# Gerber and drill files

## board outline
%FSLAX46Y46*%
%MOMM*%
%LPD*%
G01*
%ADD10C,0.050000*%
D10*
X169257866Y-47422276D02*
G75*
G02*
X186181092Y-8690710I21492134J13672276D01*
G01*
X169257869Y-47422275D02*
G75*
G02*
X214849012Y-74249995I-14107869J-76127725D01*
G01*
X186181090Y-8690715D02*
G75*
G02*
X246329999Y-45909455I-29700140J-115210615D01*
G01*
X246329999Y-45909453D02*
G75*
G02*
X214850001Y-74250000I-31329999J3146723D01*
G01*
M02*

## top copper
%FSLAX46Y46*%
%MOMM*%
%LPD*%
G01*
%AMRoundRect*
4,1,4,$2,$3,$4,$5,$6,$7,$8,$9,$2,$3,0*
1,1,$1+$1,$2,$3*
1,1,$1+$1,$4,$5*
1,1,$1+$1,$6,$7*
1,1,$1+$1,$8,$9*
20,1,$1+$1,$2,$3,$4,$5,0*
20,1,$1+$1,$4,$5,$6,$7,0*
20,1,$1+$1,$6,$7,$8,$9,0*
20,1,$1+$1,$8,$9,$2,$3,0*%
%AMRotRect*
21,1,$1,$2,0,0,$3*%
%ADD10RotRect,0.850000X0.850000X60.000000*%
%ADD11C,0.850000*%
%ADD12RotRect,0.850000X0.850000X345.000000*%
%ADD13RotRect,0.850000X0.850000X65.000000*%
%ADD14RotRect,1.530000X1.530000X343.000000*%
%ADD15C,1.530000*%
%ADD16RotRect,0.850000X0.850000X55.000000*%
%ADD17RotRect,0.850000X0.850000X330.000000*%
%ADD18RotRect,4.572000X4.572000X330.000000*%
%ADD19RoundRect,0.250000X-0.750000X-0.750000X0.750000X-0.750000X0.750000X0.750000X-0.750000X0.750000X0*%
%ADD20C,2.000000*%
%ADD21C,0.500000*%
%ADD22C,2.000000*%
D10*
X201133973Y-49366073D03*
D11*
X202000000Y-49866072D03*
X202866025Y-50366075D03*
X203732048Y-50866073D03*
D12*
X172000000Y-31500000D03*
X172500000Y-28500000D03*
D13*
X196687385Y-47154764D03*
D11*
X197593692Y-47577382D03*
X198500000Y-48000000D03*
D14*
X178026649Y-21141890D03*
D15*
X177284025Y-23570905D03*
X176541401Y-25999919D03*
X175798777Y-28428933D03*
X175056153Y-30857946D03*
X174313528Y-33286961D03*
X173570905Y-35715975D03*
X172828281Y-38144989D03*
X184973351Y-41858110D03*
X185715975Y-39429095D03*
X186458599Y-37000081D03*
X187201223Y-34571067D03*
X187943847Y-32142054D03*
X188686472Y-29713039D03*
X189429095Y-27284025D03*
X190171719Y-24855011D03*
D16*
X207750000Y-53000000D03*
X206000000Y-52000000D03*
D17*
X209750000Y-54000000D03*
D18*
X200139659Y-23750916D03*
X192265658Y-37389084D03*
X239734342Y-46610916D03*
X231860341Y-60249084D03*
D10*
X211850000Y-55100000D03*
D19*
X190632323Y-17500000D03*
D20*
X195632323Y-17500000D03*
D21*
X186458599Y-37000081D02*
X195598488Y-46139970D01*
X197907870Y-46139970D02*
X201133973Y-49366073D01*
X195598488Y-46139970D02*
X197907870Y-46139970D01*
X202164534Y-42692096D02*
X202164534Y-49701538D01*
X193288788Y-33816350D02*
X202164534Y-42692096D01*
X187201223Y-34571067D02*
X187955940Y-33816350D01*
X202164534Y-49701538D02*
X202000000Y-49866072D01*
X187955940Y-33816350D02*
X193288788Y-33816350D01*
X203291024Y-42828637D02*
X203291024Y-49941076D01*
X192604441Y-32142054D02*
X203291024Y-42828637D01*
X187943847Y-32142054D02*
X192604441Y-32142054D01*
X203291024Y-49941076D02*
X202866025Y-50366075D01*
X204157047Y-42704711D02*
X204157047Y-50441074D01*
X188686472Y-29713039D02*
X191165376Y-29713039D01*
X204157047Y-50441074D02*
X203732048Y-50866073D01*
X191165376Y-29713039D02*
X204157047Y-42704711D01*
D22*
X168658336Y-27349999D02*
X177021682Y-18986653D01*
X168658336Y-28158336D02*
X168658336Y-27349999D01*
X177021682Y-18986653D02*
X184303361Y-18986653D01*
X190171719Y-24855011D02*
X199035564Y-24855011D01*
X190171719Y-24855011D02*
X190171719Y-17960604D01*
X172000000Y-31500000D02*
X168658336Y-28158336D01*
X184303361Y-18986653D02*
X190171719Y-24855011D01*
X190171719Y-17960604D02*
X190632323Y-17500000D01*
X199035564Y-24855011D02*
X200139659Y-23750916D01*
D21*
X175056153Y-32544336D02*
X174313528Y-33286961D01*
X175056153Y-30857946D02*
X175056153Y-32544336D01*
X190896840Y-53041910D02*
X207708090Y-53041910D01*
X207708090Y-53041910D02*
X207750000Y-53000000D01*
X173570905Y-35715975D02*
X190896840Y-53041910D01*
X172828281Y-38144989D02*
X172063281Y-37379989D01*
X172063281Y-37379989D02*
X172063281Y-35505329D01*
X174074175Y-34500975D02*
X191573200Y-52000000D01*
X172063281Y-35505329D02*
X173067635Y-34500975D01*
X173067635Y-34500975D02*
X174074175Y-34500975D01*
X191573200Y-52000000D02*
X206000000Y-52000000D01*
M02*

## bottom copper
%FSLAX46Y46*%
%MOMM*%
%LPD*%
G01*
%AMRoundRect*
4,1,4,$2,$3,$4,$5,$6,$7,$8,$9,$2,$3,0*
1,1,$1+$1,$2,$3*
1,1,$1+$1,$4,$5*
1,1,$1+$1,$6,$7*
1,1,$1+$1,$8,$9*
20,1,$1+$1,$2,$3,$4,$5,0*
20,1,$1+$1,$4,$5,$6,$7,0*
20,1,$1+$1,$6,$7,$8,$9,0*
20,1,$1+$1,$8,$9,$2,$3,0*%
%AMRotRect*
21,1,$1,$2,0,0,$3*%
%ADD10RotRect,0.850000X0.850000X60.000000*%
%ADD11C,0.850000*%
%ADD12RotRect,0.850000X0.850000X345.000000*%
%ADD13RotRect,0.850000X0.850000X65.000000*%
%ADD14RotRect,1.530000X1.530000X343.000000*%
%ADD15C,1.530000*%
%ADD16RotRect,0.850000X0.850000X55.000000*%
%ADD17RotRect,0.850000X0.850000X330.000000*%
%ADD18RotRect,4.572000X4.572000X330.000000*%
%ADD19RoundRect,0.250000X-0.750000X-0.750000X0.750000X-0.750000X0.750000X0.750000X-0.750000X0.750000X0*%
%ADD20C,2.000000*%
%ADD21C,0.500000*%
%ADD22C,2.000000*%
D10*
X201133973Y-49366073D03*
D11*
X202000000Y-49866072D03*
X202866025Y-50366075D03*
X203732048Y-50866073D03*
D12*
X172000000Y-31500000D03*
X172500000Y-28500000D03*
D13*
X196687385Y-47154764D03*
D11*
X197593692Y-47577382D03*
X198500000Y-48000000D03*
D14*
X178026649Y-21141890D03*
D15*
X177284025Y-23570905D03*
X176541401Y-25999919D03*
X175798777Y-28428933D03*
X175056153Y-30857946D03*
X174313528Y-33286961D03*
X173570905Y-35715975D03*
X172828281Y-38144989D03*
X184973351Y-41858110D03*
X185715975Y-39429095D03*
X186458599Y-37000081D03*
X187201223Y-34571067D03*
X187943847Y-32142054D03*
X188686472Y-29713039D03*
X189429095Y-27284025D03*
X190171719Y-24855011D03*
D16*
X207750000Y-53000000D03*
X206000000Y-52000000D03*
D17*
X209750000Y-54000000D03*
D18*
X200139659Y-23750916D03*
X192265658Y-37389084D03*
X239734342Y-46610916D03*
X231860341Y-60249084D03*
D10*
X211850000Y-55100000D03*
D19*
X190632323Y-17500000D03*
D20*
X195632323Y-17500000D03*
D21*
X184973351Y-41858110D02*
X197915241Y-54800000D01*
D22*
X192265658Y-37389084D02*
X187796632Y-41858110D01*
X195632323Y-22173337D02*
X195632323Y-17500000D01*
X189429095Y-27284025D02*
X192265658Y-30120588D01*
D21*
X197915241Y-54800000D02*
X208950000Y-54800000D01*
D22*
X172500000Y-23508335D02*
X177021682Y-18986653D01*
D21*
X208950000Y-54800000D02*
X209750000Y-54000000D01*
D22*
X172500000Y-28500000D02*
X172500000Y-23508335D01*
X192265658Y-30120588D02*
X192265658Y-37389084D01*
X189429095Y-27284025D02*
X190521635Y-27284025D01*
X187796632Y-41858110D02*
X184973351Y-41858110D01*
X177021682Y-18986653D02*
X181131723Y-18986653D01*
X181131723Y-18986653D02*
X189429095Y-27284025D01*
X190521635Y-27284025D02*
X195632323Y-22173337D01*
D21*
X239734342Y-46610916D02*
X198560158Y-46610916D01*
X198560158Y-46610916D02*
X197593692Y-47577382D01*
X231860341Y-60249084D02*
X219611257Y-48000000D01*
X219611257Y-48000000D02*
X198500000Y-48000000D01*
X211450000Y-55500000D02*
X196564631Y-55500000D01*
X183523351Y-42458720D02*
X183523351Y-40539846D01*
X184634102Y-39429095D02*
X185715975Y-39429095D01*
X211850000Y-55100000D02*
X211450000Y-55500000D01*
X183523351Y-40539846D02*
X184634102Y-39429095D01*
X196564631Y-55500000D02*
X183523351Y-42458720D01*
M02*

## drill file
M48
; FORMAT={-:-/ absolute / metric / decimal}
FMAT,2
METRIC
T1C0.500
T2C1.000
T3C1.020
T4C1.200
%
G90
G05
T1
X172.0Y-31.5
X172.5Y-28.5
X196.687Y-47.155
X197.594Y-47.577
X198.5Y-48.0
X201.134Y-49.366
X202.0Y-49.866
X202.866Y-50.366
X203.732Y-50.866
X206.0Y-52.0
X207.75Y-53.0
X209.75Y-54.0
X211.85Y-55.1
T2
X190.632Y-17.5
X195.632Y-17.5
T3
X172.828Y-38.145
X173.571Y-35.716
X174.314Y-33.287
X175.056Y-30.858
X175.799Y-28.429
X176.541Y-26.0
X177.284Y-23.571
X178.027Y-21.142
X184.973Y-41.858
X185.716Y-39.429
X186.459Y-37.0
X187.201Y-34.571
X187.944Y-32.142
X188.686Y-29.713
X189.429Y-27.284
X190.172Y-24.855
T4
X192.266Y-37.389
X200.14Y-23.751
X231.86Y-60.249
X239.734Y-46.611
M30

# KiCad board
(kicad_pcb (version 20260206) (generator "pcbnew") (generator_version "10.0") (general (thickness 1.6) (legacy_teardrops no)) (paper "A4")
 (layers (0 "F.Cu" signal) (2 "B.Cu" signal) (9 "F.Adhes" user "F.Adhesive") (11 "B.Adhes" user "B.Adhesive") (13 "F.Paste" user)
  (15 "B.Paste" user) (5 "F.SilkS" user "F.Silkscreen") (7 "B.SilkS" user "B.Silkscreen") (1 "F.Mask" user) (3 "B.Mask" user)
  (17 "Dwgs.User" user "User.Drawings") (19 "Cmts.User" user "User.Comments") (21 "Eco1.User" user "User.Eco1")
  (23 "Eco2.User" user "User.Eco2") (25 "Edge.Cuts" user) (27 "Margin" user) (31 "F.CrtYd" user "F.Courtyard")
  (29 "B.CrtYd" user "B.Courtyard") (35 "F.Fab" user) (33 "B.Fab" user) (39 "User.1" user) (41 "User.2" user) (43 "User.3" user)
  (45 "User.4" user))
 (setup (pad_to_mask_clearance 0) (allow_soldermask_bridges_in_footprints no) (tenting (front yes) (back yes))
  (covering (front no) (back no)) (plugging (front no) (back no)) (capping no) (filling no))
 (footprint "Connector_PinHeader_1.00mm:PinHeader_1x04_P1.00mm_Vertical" (layer "F.Cu") (at 201.133973 49.366073 60)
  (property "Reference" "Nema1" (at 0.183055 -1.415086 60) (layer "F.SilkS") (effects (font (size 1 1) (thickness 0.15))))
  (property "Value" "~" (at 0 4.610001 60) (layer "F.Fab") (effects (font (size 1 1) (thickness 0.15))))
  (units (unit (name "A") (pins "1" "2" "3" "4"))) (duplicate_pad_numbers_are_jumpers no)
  (pad "1" thru_hole rect (at 0 0 60) (size 0.85 0.85) (drill 0.5) (layers "*.Cu" "*.Mask") (remove_unused_layers no) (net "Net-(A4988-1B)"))
  (pad "2" thru_hole circle (at 0.000002 1.000001 60) (size 0.85 0.85) (drill 0.5) (layers "*.Cu" "*.Mask") (remove_unused_layers no)
   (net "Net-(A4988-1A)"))
  (pad "3" thru_hole circle (at -0.000001 2.000002 60) (size 0.85 0.85) (drill 0.5) (layers "*.Cu" "*.Mask") (remove_unused_layers no)
   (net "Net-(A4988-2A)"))
  (pad "4" thru_hole circle (at -0.000001 2.999999 60) (size 0.85 0.85) (drill 0.5) (layers "*.Cu" "*.Mask") (remove_unused_layers no)
   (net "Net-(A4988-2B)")))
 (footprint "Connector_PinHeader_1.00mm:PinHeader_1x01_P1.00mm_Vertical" (layer "F.Cu") (at 172 31.5 -15)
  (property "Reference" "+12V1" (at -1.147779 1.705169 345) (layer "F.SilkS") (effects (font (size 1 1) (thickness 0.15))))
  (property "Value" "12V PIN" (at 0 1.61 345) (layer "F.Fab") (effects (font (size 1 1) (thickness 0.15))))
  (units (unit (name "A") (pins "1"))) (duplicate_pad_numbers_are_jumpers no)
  (pad "1" thru_hole rect (at 0 0 345) (size 0.85 0.85) (drill 0.5) (layers "*.Cu" "*.Mask") (remove_unused_layers no) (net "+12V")))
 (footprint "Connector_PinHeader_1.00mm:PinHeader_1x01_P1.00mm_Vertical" (layer "F.Cu") (at 172.5 28.5 -15)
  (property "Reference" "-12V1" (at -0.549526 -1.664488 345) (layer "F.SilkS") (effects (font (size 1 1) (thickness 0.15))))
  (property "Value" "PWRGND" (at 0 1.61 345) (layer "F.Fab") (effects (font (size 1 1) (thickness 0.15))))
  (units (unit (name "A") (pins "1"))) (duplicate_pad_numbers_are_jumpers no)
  (pad "1" thru_hole rect (at 0 0 345) (size 0.85 0.85) (drill 0.5) (layers "*.Cu" "*.Mask") (remove_unused_layers no) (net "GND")))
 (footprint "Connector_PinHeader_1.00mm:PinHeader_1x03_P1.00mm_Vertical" (layer "F.Cu") (at 196.687385 47.154764 65)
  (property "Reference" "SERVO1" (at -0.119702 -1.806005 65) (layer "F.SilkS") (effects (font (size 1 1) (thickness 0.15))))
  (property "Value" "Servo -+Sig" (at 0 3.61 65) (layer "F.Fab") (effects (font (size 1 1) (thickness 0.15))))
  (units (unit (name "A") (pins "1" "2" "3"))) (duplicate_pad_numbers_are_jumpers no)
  (pad "1" thru_hole rect (at 0 0 65) (size 0.85 0.85) (drill 0.5) (layers "*.Cu" "*.Mask") (remove_unused_layers no)
   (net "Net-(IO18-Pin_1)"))
  (pad "2" thru_hole circle (at 0 0.999999 65) (size 0.85 0.85) (drill 0.5) (layers "*.Cu" "*.Mask") (remove_unused_layers no)
   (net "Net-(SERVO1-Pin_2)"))
  (pad "3" thru_hole circle (at 0 1.999999 65) (size 0.85 0.85) (drill 0.5) (layers "*.Cu" "*.Mask") (remove_unused_layers no)
   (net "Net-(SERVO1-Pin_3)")))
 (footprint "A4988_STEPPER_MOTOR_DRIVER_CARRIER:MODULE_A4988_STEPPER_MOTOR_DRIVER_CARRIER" (layer "F.Cu") (at 181.5 31.5 -17)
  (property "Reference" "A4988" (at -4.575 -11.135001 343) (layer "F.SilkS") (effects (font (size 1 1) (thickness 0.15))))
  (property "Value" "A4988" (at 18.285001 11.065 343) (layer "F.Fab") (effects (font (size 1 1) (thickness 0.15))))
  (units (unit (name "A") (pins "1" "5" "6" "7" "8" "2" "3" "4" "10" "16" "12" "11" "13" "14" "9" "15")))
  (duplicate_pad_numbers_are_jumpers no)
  (pad "1" thru_hole rect (at -6.35 -8.89 343) (size 1.53 1.53) (drill 1.02) (layers "*.Cu" "*.Mask") (remove_unused_layers no)
   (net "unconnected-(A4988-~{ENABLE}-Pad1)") (solder_mask_margin 0.102))
  (pad "2" thru_hole circle (at -6.35 -6.349999 343) (size 1.53 1.53) (drill 1.02) (layers "*.Cu" "*.Mask") (remove_unused_layers no)
   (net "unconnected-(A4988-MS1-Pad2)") (solder_mask_margin 0.102))
  (pad "3" thru_hole circle (at -6.35 -3.81 343) (size 1.53 1.53) (drill 1.02) (layers "*.Cu" "*.Mask") (remove_unused_layers no)
   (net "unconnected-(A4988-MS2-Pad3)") (solder_mask_margin 0.102))
  (pad "4" thru_hole circle (at -6.35 -1.27 343) (size 1.53 1.53) (drill 1.02) (layers "*.Cu" "*.Mask") (remove_unused_layers no)
   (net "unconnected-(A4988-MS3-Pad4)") (solder_mask_margin 0.102))
  (pad "5" thru_hole circle (at -6.35 1.269999 343) (size 1.53 1.53) (drill 1.02) (layers "*.Cu" "*.Mask") (remove_unused_layers no)
   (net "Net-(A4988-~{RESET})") (solder_mask_margin 0.102))
  (pad "6" thru_hole circle (at -6.350001 3.81 343) (size 1.53 1.53) (drill 1.02) (layers "*.Cu" "*.Mask") (remove_unused_layers no)
   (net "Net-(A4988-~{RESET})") (solder_mask_margin 0.102))
  (pad "7" thru_hole circle (at -6.349999 6.35 343) (size 1.53 1.53) (drill 1.02) (layers "*.Cu" "*.Mask") (remove_unused_layers no)
   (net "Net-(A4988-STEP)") (solder_mask_margin 0.102))
  (pad "8" thru_hole circle (at -6.349999 8.89 343) (size 1.53 1.53) (drill 1.02) (layers "*.Cu" "*.Mask") (remove_unused_layers no)
   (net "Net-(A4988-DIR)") (solder_mask_margin 0.102))
  (pad "9" thru_hole circle (at 6.35 8.89 343) (size 1.53 1.53) (drill 1.02) (layers "*.Cu" "*.Mask") (remove_unused_layers no) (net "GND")
   (solder_mask_margin 0.102))
  (pad "10" thru_hole circle (at 6.35 6.349999 343) (size 1.53 1.53) (drill 1.02) (layers "*.Cu" "*.Mask") (remove_unused_layers no)
   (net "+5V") (solder_mask_margin 0.102))
  (pad "11" thru_hole circle (at 6.35 3.81 343) (size 1.53 1.53) (drill 1.02) (layers "*.Cu" "*.Mask") (remove_unused_layers no)
   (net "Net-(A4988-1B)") (solder_mask_margin 0.102))
  (pad "12" thru_hole circle (at 6.35 1.27 343) (size 1.53 1.53) (drill 1.02) (layers "*.Cu" "*.Mask") (remove_unused_layers no)
   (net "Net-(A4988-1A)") (solder_mask_margin 0.102))
  (pad "13" thru_hole circle (at 6.35 -1.269999 343) (size 1.53 1.53) (drill 1.02) (layers "*.Cu" "*.Mask") (remove_unused_layers no)
   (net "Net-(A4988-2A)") (solder_mask_margin 0.102))
  (pad "14" thru_hole circle (at 6.350001 -3.81 343) (size 1.53 1.53) (drill 1.02) (layers "*.Cu" "*.Mask") (remove_unused_layers no)
   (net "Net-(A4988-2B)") (solder_mask_margin 0.102))
  (pad "15" thru_hole circle (at 6.349999 -6.35 343) (size 1.53 1.53) (drill 1.02) (layers "*.Cu" "*.Mask") (remove_unused_layers no)
   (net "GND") (solder_mask_margin 0.102))
  (pad "16" thru_hole circle (at 6.349999 -8.89 343) (size 1.53 1.53) (drill 1.02) (layers "*.Cu" "*.Mask") (remove_unused_layers no)
   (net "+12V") (solder_mask_margin 0.102)))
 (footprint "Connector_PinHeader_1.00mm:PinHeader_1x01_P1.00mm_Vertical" (layer "F.Cu") (at 207.75 53 55)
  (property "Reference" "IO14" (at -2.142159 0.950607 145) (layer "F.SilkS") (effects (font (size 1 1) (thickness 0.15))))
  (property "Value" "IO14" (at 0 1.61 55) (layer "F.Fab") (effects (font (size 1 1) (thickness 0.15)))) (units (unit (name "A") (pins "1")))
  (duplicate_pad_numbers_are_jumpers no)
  (pad "1" thru_hole rect (at 0 0 55) (size 0.85 0.85) (drill 0.5) (layers "*.Cu" "*.Mask") (remove_unused_layers no)
   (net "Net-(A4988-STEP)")))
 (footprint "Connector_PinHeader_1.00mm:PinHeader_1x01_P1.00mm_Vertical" (layer "F.Cu") (at 206 52 55)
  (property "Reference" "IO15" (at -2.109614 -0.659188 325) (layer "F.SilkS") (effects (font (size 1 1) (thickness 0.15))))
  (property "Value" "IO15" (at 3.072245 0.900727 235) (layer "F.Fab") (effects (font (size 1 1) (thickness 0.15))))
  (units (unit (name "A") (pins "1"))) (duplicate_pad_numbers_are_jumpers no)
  (pad "1" thru_hole rect (at 0 0 55) (size 0.85 0.85) (drill 0.5) (layers "*.Cu" "*.Mask") (remove_unused_layers no)
   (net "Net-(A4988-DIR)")))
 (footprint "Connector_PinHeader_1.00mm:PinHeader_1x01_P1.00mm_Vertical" (layer "F.Cu") (at 209.75 54 -30)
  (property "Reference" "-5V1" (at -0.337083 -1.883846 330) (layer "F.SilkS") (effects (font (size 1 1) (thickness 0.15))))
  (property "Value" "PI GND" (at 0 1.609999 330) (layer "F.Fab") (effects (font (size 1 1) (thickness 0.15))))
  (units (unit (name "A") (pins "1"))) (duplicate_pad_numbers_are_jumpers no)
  (pad "1" thru_hole rect (at 0 0 330) (size 0.85 0.85) (drill 0.5) (layers "*.Cu" "*.Mask") (remove_unused_layers no) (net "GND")))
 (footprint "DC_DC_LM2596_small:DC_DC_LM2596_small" (layer "F.Cu") (at 216 42 -30)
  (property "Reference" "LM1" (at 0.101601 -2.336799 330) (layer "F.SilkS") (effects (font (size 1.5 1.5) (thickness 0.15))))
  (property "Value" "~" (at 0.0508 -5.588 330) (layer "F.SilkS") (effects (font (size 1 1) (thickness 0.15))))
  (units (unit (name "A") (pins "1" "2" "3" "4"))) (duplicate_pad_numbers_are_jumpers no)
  (pad "1" thru_hole rect (at -22.86 -7.874 330) (size 4.572 4.572) (drill 1.2) (layers "*.Cu" "*.Mask" "F.SilkS") (remove_unused_layers no)
   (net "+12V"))
  (pad "2" thru_hole rect (at -22.860001 7.874001 330) (size 4.572 4.572) (drill 1.2) (layers "*.Cu" "*.Mask" "F.SilkS")
   (remove_unused_layers no) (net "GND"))
  (pad "3" thru_hole rect (at 22.860001 -7.874001 330) (size 4.572 4.572) (drill 1.2) (layers "*.Cu" "*.Mask" "F.SilkS")
   (remove_unused_layers no) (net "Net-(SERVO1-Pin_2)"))
  (pad "4" thru_hole rect (at 22.86 7.874 330) (size 4.572 4.572) (drill 1.2) (layers "*.Cu" "*.Mask" "F.SilkS") (remove_unused_layers no)
   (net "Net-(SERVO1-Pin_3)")))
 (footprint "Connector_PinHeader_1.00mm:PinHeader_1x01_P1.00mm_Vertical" (layer "F.Cu") (at 211.85 55.1 60)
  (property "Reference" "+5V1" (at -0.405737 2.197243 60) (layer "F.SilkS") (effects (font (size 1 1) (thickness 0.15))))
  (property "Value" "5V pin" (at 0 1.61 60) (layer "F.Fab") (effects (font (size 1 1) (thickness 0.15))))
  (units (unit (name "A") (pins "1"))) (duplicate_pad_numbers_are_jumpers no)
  (pad "1" thru_hole rect (at 0 0 60) (size 0.85 0.85) (drill 0.5) (layers "*.Cu" "*.Mask") (remove_unused_layers no) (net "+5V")))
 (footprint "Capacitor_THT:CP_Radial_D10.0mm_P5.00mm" (layer "F.Cu") (at 190.632323 17.5)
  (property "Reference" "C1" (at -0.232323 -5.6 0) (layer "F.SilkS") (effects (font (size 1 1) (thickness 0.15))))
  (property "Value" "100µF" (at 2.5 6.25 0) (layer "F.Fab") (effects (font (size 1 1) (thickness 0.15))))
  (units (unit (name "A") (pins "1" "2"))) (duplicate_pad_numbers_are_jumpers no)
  (pad "1" thru_hole roundrect (at 0 0) (size 2 2) (drill 1) (layers "*.Cu" "*.Mask") (remove_unused_layers no) (roundrect_rratio 0.125)
   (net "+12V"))
  (pad "2" thru_hole circle (at 5 0) (size 2 2) (drill 1) (layers "*.Cu" "*.Mask") (remove_unused_layers no) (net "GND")))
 (gr_arc (start 169.257866 47.422276) (mid 167.408448 23.55123) (end 186.181092 8.69071) (stroke (width 0.05) (type default))
  (layer "Edge.Cuts"))
 (gr_arc (start 169.257869 47.422275) (mid 194.415705 56.821693) (end 214.849012 74.249995) (stroke (width 0.05) (type default))
  (layer "Edge.Cuts"))
 (gr_arc (start 186.18109 8.690715) (mid 219.085349 22.72686) (end 246.329999 45.909455) (stroke (width 0.05) (type default))
  (layer "Edge.Cuts"))
 (gr_arc (start 246.329999 45.909453) (mid 236.067623 66.164139) (end 214.850001 74.250001) (stroke (width 0.05) (type default))
  (layer "Edge.Cuts"))
 (segment (start 186.458599 37.000081) (end 195.598488 46.13997) (width 0.5) (layer "F.Cu") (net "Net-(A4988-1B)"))
 (segment (start 197.90787 46.13997) (end 201.133973 49.366073) (width 0.5) (layer "F.Cu") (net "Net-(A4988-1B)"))
 (segment (start 195.598488 46.13997) (end 197.90787 46.13997) (width 0.5) (layer "F.Cu") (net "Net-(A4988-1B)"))
 (segment (start 202.164534 42.692096) (end 202.164534 49.701538) (width 0.5) (layer "F.Cu") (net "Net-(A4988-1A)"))
 (segment (start 193.288788 33.81635) (end 202.164534 42.692096) (width 0.5) (layer "F.Cu") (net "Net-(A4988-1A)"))
 (segment (start 187.201223 34.571067) (end 187.95594 33.81635) (width 0.5) (layer "F.Cu") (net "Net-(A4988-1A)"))
 (segment (start 202.164534 49.701538) (end 202 49.866072) (width 0.5) (layer "F.Cu") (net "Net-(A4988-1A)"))
 (segment (start 187.95594 33.81635) (end 193.288788 33.81635) (width 0.5) (layer "F.Cu") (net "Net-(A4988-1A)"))
 (segment (start 203.291024 42.828637) (end 203.291024 49.941076) (width 0.5) (layer "F.Cu") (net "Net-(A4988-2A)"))
 (segment (start 192.604441 32.142054) (end 203.291024 42.828637) (width 0.5) (layer "F.Cu") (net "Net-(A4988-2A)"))
 (segment (start 187.943847 32.142054) (end 192.604441 32.142054) (width 0.5) (layer "F.Cu") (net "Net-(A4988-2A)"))
 (segment (start 203.291024 49.941076) (end 202.866025 50.366075) (width 0.5) (layer "F.Cu") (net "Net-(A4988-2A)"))
 (segment (start 204.157047 42.704711) (end 204.157047 50.441074) (width 0.5) (layer "F.Cu") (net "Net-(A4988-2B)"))
 (segment (start 188.686472 29.713039) (end 191.165376 29.713039) (width 0.5) (layer "F.Cu") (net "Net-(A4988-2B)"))
 (segment (start 204.157047 50.441074) (end 203.732048 50.866073) (width 0.5) (layer "F.Cu") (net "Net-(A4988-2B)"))
 (segment (start 191.165376 29.713039) (end 204.157047 42.704711) (width 0.5) (layer "F.Cu") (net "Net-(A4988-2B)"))
 (segment (start 168.658336 27.349999) (end 177.021682 18.986653) (width 2) (layer "F.Cu") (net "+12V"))
 (segment (start 168.658336 28.158336) (end 168.658336 27.349999) (width 2) (layer "F.Cu") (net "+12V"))
 (segment (start 177.021682 18.986653) (end 184.303361 18.986653) (width 2) (layer "F.Cu") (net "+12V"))
 (segment (start 190.171719 24.855011) (end 199.035564 24.855011) (width 2) (layer "F.Cu") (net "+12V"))
 (segment (start 190.171719 24.855011) (end 190.171719 17.960604) (width 2) (layer "F.Cu") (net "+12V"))
 (segment (start 172 31.5) (end 168.658336 28.158336) (width 2) (layer "F.Cu") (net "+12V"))
 (segment (start 184.303361 18.986653) (end 190.171719 24.855011) (width 2) (layer "F.Cu") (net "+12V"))
 (segment (start 190.171719 17.960604) (end 190.632323 17.5) (width 2) (layer "F.Cu") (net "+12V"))
 (segment (start 199.035564 24.855011) (end 200.139659 23.750916) (width 2) (layer "F.Cu") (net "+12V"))
 (segment (start 184.973351 41.85811) (end 197.915241 54.8) (width 0.5) (layer "B.Cu") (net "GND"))
 (segment (start 192.265658 37.389084) (end 187.796632 41.85811) (width 2) (layer "B.Cu") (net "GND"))
 (segment (start 195.632323 22.173337) (end 195.632323 17.5) (width 2) (layer "B.Cu") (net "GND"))
 (segment (start 189.429095 27.284025) (end 192.265658 30.120588) (width 2) (layer "B.Cu") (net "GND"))
 (segment (start 197.915241 54.8) (end 208.95 54.8) (width 0.5) (layer "B.Cu") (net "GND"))
 (segment (start 172.5 23.508335) (end 177.021682 18.986653) (width 2) (layer "B.Cu") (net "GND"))
 (segment (start 208.95 54.8) (end 209.75 54) (width 0.5) (layer "B.Cu") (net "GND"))
 (segment (start 172.5 28.5) (end 172.5 23.508335) (width 2) (layer "B.Cu") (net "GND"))
 (segment (start 192.265658 30.120588) (end 192.265658 37.389084) (width 2) (layer "B.Cu") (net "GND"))
 (segment (start 189.429095 27.284025) (end 190.521635 27.284025) (width 2) (layer "B.Cu") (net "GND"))
 (segment (start 187.796632 41.85811) (end 184.973351 41.85811) (width 2) (layer "B.Cu") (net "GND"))
 (segment (start 177.021682 18.986653) (end 181.131723 18.986653) (width 2) (layer "B.Cu") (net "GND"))
 (segment (start 181.131723 18.986653) (end 189.429095 27.284025) (width 2) (layer "B.Cu") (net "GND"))
 (segment (start 190.521635 27.284025) (end 195.632323 22.173337) (width 2) (layer "B.Cu") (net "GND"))
 (segment (start 239.734342 46.610916) (end 198.560158 46.610916) (width 0.5) (layer "B.Cu") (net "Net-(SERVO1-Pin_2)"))
 (segment (start 198.560158 46.610916) (end 197.593692 47.577382) (width 0.5) (layer "B.Cu") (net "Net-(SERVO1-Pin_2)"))
 (segment (start 231.860341 60.249084) (end 219.611257 48) (width 0.5) (layer "B.Cu") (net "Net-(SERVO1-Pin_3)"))
 (segment (start 219.611257 48) (end 198.5 48) (width 0.5) (layer "B.Cu") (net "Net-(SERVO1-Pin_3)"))
 (segment (start 175.056153 32.544336) (end 174.313528 33.286961) (width 0.5) (layer "F.Cu") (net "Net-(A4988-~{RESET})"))
 (segment (start 175.056153 30.857946) (end 175.056153 32.544336) (width 0.5) (layer "F.Cu") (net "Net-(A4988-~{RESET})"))
 (segment (start 190.89684 53.04191) (end 207.70809 53.04191) (width 0.5) (layer "F.Cu") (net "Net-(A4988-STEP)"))
 (segment (start 207.70809 53.04191) (end 207.75 53) (width 0.5) (layer "F.Cu") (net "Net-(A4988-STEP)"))
 (segment (start 173.570905 35.715975) (end 190.89684 53.04191) (width 0.5) (layer "F.Cu") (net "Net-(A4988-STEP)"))
 (segment (start 172.828281 38.144989) (end 172.063281 37.379989) (width 0.5) (layer "F.Cu") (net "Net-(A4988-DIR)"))
 (segment (start 172.063281 37.379989) (end 172.063281 35.505329) (width 0.5) (layer "F.Cu") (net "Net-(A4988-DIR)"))
 (segment (start 174.074175 34.500975) (end 191.5732 52) (width 0.5) (layer "F.Cu") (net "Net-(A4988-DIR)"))
 (segment (start 172.063281 35.505329) (end 173.067635 34.500975) (width 0.5) (layer "F.Cu") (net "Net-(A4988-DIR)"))
 (segment (start 173.067635 34.500975) (end 174.074175 34.500975) (width 0.5) (layer "F.Cu") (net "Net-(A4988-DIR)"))
 (segment (start 191.5732 52) (end 206 52) (width 0.5) (layer "F.Cu") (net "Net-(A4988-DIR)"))
 (segment (start 211.45 55.5) (end 196.564631 55.5) (width 0.5) (layer "B.Cu") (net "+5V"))
 (segment (start 183.523351 42.45872) (end 183.523351 40.539846) (width 0.5) (layer "B.Cu") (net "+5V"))
 (segment (start 184.634102 39.429095) (end 185.715975 39.429095) (width 0.5) (layer "B.Cu") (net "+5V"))
 (segment (start 211.85 55.1) (end 211.45 55.5) (width 0.5) (layer "B.Cu") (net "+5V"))
 (segment (start 183.523351 40.539846) (end 184.634102 39.429095) (width 0.5) (layer "B.Cu") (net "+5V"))
 (segment (start 196.564631 55.5) (end 183.523351 42.45872) (width 0.5) (layer "B.Cu") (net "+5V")))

